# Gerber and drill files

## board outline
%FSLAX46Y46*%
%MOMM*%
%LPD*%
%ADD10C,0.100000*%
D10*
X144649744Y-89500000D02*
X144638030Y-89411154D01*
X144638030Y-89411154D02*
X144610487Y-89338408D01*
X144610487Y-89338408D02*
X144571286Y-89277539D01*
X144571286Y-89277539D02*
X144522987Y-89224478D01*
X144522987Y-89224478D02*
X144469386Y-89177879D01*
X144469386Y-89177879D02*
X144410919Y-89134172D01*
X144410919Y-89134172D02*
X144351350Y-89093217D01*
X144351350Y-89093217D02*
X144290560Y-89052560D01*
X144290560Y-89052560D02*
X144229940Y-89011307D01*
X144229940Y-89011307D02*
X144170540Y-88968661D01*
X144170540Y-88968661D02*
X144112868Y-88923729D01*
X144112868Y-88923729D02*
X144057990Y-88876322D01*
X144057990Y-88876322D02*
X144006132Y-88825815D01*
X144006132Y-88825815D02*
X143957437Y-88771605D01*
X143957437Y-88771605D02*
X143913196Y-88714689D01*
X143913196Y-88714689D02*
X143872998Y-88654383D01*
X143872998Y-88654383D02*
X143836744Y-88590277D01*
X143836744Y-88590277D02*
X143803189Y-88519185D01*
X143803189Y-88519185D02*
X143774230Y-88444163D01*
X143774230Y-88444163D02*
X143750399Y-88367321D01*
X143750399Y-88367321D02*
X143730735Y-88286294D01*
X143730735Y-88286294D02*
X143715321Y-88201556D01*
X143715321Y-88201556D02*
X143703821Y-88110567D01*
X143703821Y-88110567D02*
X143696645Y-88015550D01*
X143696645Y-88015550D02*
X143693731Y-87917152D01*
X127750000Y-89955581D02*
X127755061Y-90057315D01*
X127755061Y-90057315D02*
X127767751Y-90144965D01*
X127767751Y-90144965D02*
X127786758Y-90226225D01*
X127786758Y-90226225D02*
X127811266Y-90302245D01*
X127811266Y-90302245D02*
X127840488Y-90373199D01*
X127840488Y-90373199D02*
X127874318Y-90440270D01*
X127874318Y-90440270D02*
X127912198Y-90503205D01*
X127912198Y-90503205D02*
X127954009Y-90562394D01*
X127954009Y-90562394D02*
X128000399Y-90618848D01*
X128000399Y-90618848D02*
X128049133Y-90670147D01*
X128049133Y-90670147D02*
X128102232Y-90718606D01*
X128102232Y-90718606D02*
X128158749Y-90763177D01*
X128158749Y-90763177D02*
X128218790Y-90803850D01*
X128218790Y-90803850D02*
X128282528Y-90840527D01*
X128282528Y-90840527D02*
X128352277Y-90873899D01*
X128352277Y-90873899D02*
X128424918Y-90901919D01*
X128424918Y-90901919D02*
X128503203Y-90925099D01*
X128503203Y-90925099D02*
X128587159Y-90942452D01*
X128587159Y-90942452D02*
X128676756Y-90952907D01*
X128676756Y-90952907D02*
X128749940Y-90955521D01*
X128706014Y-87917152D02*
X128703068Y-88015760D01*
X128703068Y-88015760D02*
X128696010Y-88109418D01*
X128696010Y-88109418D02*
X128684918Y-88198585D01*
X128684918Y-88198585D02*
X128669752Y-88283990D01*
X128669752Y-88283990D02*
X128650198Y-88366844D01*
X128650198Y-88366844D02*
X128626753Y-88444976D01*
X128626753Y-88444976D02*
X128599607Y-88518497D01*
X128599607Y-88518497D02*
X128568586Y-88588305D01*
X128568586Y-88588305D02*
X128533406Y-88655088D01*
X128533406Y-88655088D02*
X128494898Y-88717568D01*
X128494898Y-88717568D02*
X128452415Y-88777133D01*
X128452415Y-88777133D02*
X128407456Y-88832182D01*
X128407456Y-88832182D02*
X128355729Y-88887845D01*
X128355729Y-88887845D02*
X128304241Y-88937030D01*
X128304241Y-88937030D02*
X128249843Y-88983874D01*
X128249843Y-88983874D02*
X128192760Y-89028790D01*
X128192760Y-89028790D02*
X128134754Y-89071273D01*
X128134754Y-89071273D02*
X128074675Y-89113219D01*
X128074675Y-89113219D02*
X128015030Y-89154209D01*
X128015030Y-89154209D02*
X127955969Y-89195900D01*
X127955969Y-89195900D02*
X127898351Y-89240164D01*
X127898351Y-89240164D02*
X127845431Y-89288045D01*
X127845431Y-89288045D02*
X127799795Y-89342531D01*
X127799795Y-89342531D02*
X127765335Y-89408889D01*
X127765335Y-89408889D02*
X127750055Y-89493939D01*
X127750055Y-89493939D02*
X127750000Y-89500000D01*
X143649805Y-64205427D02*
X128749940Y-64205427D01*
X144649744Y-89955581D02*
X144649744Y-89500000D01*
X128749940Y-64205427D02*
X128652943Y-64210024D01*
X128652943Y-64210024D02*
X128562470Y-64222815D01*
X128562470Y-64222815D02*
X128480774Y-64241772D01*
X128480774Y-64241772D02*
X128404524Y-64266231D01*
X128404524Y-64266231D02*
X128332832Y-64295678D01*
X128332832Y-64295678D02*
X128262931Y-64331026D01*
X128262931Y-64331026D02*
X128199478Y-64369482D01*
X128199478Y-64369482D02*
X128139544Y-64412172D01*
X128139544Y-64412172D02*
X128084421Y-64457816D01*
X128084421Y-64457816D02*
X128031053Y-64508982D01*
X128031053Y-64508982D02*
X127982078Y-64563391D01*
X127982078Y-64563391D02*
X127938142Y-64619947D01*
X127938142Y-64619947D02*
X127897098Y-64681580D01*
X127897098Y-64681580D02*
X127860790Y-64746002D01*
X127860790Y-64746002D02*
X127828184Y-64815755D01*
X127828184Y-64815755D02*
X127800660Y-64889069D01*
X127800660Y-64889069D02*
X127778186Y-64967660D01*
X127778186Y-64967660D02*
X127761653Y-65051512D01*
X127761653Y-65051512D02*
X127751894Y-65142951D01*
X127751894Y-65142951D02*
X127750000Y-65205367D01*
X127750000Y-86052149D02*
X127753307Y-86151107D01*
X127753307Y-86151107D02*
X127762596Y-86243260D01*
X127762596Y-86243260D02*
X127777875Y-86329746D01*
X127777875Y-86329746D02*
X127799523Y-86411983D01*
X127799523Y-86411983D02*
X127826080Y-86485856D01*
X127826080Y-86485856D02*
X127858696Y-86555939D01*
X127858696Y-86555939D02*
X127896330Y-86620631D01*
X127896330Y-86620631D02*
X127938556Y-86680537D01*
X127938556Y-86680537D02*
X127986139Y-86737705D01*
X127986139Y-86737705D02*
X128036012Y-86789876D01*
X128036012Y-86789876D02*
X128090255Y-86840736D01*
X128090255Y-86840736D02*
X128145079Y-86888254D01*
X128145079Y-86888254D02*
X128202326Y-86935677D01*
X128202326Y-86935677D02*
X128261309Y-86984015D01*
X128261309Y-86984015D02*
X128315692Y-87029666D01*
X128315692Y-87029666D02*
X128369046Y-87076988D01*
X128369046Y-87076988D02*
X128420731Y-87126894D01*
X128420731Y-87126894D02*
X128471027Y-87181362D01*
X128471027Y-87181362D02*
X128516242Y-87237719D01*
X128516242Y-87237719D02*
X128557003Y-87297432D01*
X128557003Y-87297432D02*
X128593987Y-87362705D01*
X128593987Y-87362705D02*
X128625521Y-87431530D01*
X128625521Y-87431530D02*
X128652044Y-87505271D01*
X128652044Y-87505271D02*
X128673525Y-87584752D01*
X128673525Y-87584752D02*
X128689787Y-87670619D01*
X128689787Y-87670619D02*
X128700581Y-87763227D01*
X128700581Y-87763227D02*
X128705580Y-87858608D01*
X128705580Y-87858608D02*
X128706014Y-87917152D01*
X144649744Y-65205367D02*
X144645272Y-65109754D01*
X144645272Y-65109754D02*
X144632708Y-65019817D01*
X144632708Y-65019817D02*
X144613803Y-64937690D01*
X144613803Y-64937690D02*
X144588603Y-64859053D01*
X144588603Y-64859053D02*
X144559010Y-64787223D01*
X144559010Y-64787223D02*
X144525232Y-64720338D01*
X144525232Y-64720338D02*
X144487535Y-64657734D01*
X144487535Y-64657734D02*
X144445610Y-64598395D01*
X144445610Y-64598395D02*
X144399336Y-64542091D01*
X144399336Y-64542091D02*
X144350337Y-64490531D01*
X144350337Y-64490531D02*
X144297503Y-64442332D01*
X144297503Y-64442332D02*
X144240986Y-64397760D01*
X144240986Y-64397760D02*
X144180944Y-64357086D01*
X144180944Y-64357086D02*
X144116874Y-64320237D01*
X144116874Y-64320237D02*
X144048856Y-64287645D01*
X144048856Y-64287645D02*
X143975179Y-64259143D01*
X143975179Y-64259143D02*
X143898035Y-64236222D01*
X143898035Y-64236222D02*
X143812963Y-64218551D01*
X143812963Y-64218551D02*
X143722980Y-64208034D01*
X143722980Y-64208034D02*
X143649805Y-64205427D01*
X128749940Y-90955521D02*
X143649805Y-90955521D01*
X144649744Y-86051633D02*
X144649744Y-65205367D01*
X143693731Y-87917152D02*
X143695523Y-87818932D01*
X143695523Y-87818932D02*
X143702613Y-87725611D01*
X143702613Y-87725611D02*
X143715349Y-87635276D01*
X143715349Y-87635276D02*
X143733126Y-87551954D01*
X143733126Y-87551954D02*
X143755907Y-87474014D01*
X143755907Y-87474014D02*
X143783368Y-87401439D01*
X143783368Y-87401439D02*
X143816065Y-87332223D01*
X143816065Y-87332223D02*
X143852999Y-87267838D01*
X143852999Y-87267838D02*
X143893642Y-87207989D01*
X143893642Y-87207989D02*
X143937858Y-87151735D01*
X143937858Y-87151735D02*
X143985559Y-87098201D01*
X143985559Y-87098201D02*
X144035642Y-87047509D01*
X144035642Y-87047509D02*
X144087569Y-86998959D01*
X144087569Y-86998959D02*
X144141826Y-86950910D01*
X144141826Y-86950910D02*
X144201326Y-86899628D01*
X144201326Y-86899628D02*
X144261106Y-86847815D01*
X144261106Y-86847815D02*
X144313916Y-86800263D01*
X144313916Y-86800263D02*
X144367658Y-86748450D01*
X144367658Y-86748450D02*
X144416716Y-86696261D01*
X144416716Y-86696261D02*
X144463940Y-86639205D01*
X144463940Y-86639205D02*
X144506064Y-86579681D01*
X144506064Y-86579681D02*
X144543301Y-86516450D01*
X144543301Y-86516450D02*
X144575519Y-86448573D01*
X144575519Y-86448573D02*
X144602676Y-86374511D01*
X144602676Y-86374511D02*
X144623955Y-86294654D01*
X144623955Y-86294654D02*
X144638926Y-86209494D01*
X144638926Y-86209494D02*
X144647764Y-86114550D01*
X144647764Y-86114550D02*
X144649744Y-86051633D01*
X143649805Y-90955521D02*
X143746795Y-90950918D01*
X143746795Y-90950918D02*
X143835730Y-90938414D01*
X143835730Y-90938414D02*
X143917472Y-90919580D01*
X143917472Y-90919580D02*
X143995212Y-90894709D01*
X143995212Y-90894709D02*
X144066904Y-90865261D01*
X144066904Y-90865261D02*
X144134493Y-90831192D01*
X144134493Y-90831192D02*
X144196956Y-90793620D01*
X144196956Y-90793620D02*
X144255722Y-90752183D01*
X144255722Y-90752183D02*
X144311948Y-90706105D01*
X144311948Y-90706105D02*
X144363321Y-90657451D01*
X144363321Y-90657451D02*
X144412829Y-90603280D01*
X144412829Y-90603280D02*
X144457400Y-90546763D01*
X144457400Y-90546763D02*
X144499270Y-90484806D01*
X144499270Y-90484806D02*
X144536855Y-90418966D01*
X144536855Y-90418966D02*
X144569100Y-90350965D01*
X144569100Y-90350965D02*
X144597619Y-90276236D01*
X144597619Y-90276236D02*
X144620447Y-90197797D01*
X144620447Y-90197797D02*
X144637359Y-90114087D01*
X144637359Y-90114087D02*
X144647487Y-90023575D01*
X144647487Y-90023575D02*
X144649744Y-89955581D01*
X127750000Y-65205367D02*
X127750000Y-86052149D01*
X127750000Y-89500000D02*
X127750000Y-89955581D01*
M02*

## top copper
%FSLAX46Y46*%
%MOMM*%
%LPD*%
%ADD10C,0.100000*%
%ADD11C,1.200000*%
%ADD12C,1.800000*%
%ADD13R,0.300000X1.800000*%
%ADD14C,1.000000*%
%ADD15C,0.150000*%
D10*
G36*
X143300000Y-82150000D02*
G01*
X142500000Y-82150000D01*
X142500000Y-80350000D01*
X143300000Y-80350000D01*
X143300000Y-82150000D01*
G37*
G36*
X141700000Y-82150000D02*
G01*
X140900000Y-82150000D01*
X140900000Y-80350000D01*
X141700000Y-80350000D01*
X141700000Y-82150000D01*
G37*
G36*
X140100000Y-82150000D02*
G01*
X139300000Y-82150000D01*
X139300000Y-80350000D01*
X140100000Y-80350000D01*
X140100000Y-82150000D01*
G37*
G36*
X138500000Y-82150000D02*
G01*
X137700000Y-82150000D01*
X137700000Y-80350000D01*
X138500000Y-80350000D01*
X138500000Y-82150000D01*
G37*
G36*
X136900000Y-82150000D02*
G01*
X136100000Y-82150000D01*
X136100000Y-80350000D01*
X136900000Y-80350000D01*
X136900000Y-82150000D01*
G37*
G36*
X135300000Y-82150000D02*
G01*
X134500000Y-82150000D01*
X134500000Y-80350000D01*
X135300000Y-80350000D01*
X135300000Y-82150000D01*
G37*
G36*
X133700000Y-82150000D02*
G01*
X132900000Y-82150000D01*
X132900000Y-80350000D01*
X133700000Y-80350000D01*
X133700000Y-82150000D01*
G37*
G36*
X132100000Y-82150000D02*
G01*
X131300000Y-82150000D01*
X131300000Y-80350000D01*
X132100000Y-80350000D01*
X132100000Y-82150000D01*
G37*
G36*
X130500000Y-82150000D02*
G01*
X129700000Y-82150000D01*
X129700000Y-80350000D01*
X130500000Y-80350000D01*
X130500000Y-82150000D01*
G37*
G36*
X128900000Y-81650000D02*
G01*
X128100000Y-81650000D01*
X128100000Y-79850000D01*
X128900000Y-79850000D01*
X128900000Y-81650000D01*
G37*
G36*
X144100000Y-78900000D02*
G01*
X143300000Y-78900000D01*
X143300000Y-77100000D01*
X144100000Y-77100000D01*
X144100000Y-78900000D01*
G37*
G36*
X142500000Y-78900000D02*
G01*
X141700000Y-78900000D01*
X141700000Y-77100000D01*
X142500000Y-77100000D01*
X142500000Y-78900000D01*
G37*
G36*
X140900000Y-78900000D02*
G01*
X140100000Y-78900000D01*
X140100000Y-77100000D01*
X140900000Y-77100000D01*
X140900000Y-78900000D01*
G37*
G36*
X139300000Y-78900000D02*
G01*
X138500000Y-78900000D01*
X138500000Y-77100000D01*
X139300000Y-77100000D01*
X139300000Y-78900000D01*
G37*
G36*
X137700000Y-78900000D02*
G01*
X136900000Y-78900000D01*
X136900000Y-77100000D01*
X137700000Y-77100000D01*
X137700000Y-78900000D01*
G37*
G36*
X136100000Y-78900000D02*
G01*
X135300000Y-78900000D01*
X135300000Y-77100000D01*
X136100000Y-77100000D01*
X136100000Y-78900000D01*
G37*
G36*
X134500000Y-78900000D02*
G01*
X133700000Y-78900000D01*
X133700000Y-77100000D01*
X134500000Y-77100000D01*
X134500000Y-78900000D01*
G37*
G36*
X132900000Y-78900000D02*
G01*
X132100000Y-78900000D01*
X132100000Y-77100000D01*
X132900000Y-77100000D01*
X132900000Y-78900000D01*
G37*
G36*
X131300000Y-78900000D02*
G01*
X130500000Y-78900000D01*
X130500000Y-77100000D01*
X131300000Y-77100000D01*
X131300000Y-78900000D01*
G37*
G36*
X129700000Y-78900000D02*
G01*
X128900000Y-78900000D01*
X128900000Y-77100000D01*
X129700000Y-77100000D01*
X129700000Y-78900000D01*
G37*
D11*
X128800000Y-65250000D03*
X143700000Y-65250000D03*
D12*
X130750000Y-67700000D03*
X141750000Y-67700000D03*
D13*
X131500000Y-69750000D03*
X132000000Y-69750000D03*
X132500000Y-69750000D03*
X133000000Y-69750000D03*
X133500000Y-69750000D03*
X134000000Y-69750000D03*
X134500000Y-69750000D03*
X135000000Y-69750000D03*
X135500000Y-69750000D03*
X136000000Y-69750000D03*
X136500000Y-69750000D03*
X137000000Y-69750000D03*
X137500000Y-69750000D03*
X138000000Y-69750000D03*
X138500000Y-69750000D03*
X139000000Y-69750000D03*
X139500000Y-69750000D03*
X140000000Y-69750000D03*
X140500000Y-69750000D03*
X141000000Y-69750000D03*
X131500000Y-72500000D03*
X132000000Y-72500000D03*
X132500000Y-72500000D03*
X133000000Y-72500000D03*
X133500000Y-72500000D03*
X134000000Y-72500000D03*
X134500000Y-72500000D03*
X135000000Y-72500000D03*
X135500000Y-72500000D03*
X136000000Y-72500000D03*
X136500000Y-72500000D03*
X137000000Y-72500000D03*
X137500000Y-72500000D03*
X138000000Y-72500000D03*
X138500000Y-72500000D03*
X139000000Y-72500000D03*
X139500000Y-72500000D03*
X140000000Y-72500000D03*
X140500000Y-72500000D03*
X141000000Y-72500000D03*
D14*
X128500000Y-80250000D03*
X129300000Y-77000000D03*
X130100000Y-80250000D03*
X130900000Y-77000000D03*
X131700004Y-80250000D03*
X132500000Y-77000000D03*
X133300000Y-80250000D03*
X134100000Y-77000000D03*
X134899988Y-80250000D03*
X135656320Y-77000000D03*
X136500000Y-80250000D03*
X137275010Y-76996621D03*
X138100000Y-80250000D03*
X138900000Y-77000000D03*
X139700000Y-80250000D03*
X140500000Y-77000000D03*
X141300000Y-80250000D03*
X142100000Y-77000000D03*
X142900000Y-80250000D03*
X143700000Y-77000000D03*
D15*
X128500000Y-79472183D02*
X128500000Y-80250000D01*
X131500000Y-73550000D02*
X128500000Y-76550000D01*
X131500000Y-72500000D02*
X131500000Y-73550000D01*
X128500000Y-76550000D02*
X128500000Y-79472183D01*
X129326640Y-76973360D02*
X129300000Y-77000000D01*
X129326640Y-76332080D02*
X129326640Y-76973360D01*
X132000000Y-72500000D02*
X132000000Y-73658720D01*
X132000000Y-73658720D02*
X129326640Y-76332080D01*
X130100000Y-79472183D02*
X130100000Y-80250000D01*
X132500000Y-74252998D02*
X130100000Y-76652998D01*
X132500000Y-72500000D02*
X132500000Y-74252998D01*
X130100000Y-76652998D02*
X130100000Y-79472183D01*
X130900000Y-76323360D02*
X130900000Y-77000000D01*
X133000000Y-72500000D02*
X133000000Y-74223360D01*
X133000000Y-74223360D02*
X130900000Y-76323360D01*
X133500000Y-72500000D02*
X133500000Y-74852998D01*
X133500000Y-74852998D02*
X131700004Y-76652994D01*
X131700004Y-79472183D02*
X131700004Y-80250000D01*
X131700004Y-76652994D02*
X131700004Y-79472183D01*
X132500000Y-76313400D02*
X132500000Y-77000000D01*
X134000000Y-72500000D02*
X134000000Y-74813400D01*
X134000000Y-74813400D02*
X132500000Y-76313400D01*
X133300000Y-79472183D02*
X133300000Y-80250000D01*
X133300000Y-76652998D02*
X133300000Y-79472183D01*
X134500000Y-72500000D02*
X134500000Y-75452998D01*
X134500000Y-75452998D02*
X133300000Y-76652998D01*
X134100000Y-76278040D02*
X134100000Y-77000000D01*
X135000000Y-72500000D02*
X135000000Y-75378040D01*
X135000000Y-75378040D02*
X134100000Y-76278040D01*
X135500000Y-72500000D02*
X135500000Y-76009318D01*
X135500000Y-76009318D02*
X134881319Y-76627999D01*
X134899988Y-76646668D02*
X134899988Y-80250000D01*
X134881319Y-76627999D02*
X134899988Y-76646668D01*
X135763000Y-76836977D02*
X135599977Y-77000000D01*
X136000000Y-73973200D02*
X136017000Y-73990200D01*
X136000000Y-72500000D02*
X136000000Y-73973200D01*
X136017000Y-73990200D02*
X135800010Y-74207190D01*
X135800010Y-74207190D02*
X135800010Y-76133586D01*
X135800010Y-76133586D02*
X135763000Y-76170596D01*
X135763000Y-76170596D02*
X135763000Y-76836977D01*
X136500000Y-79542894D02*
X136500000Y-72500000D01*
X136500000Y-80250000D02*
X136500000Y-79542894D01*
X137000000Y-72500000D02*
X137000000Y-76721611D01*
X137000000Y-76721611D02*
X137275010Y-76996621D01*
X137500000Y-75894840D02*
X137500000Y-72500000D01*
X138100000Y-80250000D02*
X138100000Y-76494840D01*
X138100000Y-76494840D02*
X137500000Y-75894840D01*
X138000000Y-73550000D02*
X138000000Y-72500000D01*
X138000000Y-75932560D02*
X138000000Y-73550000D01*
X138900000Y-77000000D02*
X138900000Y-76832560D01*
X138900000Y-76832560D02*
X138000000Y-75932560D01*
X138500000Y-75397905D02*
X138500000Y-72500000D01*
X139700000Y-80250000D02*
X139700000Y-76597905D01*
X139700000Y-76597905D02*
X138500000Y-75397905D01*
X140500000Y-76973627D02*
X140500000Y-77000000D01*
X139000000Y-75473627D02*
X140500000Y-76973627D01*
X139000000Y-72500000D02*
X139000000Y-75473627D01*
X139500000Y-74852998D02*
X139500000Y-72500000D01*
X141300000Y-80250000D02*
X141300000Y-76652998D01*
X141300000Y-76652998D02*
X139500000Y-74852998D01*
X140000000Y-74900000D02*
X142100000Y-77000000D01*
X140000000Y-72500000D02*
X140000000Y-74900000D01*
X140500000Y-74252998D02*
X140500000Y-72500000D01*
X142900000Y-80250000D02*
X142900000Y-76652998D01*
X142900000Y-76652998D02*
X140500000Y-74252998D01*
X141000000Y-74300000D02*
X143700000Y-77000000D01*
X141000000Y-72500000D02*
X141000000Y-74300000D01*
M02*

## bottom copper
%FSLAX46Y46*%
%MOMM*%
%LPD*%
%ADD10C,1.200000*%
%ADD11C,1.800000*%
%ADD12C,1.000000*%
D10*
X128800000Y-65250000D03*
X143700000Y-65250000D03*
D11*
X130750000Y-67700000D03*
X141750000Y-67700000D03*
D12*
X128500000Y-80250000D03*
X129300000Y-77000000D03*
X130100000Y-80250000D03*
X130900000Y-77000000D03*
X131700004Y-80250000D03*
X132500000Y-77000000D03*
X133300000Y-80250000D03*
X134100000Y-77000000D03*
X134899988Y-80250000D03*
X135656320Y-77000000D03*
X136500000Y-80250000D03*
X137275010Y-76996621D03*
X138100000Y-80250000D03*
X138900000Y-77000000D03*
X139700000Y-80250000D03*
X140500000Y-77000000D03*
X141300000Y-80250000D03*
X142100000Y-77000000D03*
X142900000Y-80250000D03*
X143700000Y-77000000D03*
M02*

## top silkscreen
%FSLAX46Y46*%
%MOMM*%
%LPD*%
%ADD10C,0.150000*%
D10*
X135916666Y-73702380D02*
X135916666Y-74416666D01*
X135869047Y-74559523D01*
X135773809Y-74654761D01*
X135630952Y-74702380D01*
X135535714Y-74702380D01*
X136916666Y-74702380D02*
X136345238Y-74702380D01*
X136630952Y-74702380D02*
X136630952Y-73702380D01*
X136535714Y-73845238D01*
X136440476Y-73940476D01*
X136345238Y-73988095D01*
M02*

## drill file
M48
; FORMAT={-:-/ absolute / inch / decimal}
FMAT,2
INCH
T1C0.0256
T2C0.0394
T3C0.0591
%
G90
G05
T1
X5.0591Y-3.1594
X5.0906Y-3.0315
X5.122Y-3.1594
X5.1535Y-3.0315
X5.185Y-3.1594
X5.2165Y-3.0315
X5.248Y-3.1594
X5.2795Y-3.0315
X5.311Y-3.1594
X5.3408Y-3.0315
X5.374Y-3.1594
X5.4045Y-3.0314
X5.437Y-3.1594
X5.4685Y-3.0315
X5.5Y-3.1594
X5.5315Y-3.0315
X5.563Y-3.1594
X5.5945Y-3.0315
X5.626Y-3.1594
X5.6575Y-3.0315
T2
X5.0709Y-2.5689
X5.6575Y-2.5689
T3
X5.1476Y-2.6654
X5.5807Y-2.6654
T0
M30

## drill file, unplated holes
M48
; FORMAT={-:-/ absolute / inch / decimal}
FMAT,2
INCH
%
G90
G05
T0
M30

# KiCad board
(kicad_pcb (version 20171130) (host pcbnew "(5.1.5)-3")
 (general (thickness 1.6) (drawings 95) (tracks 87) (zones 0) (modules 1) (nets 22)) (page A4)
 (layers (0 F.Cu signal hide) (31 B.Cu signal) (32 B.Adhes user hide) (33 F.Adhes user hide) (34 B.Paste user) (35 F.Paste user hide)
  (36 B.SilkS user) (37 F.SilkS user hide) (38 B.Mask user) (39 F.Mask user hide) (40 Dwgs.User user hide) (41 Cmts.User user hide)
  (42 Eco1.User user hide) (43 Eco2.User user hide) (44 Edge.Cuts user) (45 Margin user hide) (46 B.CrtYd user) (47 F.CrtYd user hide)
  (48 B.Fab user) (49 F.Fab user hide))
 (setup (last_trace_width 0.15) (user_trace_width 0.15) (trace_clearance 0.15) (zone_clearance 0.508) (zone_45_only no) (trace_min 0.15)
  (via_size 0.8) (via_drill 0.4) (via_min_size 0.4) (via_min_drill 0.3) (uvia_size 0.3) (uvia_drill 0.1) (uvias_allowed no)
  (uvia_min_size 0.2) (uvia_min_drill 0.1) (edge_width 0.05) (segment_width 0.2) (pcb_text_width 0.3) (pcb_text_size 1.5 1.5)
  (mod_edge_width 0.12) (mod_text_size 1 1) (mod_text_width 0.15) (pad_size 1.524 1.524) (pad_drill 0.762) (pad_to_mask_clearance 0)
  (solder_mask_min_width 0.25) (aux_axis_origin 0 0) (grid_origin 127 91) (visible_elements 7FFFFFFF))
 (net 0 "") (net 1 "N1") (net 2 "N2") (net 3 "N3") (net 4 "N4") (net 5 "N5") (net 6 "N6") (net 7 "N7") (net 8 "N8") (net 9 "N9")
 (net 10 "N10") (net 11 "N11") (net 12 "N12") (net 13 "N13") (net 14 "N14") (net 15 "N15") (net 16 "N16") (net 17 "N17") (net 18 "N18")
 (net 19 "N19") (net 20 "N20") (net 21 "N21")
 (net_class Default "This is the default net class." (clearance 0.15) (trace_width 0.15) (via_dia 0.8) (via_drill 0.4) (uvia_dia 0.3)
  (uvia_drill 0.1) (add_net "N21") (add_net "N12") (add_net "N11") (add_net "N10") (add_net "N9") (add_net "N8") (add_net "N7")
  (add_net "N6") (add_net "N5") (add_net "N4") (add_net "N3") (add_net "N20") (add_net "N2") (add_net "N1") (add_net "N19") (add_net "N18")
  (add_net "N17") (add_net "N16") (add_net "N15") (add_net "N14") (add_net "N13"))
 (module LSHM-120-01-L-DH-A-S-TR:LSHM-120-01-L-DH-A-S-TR (layer F.Cu) (at 136.25 69.75 180)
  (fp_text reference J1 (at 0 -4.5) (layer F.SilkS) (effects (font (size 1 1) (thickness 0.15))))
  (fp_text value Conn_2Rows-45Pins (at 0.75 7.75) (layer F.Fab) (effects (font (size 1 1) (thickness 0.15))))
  (pad 44 thru_hole circle (at 7.45 4.5 270) (size 1.2 1.2) (drill 1) (layers *.Cu *.Mask) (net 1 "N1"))
  (pad 43 thru_hole circle (at -7.45 4.5 270) (size 1.2 1.2) (drill 1) (layers *.Cu *.Mask) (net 1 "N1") (solder_paste_margin -0.5))
  (pad 42 thru_hole circle (at 5.5 2.05 270) (size 1.8 1.8) (drill 1.5) (layers *.Cu *.Mask) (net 1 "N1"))
  (pad 41 thru_hole circle (at -5.5 2.05 270) (size 1.8 1.8) (drill 1.5) (layers *.Cu *.Mask) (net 1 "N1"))
  (pad 40 smd rect (at 4.75 0 270) (size 1.8 0.3) (layers F.Cu F.Paste F.Mask) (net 1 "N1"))
  (pad 39 smd rect (at 4.25 0 270) (size 1.8 0.3) (layers F.Cu F.Paste F.Mask) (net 1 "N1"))
  (pad 38 smd rect (at 3.75 0 270) (size 1.8 0.3) (layers F.Cu F.Paste F.Mask) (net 1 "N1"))
  (pad 37 smd rect (at 3.25 0 270) (size 1.8 0.3) (layers F.Cu F.Paste F.Mask) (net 1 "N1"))
  (pad 36 smd rect (at 2.75 0 270) (size 1.8 0.3) (layers F.Cu F.Paste F.Mask) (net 1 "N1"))
  (pad 35 smd rect (at 2.25 0 270) (size 1.8 0.3) (layers F.Cu F.Paste F.Mask) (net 1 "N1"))
  (pad 34 smd rect (at 1.75 0 270) (size 1.8 0.3) (layers F.Cu F.Paste F.Mask) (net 1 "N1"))
  (pad 33 smd rect (at 1.25 0 270) (size 1.8 0.3) (layers F.Cu F.Paste F.Mask) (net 1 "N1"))
  (pad 32 smd rect (at 0.75 0 270) (size 1.8 0.3) (layers F.Cu F.Paste F.Mask) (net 1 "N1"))
  (pad 31 smd rect (at 0.25 0 270) (size 1.8 0.3) (layers F.Cu F.Paste F.Mask) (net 1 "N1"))
  (pad 30 smd rect (at -0.25 0 270) (size 1.8 0.3) (layers F.Cu F.Paste F.Mask) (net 1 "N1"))
  (pad 29 smd rect (at -0.75 0 270) (size 1.8 0.3) (layers F.Cu F.Paste F.Mask) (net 1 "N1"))
  (pad 28 smd rect (at -1.25 0 270) (size 1.8 0.3) (layers F.Cu F.Paste F.Mask) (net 1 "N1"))
  (pad 27 smd rect (at -1.75 0 270) (size 1.8 0.3) (layers F.Cu F.Paste F.Mask) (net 1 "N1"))
  (pad 26 smd rect (at -2.25 0 270) (size 1.8 0.3) (layers F.Cu F.Paste F.Mask) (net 1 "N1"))
  (pad 25 smd rect (at -2.75 0 270) (size 1.8 0.3) (layers F.Cu F.Paste F.Mask) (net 1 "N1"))
  (pad 24 smd rect (at -3.25 0 270) (size 1.8 0.3) (layers F.Cu F.Paste F.Mask) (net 1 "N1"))
  (pad 23 smd rect (at -3.75 0 270) (size 1.8 0.3) (layers F.Cu F.Paste F.Mask) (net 1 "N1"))
  (pad 22 smd rect (at -4.25 0 270) (size 1.8 0.3) (layers F.Cu F.Paste F.Mask) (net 1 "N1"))
  (pad 21 smd rect (at -4.75 0 270) (size 1.8 0.3) (layers F.Cu F.Paste F.Mask) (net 1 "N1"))
  (pad 20 smd rect (at 4.75 -2.75 270) (size 1.8 0.3) (layers F.Cu F.Paste F.Mask) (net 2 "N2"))
  (pad 19 smd rect (at 4.25 -2.75 270) (size 1.8 0.3) (layers F.Cu F.Paste F.Mask) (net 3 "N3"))
  (pad 18 smd rect (at 3.75 -2.75 270) (size 1.8 0.3) (layers F.Cu F.Paste F.Mask) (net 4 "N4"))
  (pad 17 smd rect (at 3.25 -2.75 270) (size 1.8 0.3) (layers F.Cu F.Paste F.Mask) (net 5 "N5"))
  (pad 16 smd rect (at 2.75 -2.75 270) (size 1.8 0.3) (layers F.Cu F.Paste F.Mask) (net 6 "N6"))
  (pad 15 smd rect (at 2.25 -2.75 270) (size 1.8 0.3) (layers F.Cu F.Paste F.Mask) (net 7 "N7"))
  (pad 14 smd rect (at 1.75 -2.75 270) (size 1.8 0.3) (layers F.Cu F.Paste F.Mask) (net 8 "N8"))
  (pad 13 smd rect (at 1.25 -2.75 270) (size 1.8 0.3) (layers F.Cu F.Paste F.Mask) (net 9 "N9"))
  (pad 12 smd rect (at 0.75 -2.75 270) (size 1.8 0.3) (layers F.Cu F.Paste F.Mask) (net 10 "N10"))
  (pad 11 smd rect (at 0.25 -2.75 270) (size 1.8 0.3) (layers F.Cu F.Paste F.Mask) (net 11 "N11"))
  (pad 10 smd rect (at -0.25 -2.75 270) (size 1.8 0.3) (layers F.Cu F.Paste F.Mask) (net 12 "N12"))
  (pad 9 smd rect (at -0.75 -2.75 270) (size 1.8 0.3) (layers F.Cu F.Paste F.Mask) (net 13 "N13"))
  (pad 8 smd rect (at -1.25 -2.75 270) (size 1.8 0.3) (layers F.Cu F.Paste F.Mask) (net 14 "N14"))
  (pad 7 smd rect (at -1.75 -2.75 270) (size 1.8 0.3) (layers F.Cu F.Paste F.Mask) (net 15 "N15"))
  (pad 6 smd rect (at -2.25 -2.75 270) (size 1.8 0.3) (layers F.Cu F.Paste F.Mask) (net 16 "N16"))
  (pad 5 smd rect (at -2.75 -2.75 270) (size 1.8 0.3) (layers F.Cu F.Paste F.Mask) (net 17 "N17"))
  (pad 4 smd rect (at -3.25 -2.75 270) (size 1.8 0.3) (layers F.Cu F.Paste F.Mask) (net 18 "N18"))
  (pad 3 smd rect (at -3.75 -2.75 270) (size 1.8 0.3) (layers F.Cu F.Paste F.Mask) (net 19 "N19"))
  (pad 2 smd rect (at -4.25 -2.75 270) (size 1.8 0.3) (layers F.Cu F.Paste F.Mask) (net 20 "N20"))
  (pad 1 smd rect (at -4.75 -2.75 270) (size 1.8 0.3) (layers F.Cu F.Paste F.Mask) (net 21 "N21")))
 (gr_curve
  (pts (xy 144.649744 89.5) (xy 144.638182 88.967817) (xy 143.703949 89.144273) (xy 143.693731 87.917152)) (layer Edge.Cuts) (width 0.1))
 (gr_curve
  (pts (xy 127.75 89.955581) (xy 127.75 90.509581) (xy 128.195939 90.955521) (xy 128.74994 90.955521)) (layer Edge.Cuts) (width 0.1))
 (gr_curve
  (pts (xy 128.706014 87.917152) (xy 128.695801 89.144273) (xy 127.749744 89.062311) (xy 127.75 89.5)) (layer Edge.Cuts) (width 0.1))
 (gr_line (start 143.649805 64.205427) (end 128.74994 64.205427) (layer Edge.Cuts) (width 0.1))
 (gr_line (start 144.649744 89.955581) (end 144.649744 89.5) (layer Edge.Cuts) (width 0.1))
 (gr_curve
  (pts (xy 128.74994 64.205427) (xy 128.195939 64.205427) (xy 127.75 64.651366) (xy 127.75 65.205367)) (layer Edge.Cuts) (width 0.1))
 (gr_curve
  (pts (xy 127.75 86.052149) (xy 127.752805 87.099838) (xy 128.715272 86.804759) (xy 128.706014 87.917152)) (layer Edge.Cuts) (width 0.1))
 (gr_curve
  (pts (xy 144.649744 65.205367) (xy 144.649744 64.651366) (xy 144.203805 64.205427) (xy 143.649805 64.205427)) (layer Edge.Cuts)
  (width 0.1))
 (gr_line (start 128.74994 90.955521) (end 143.649805 90.955521) (layer Edge.Cuts) (width 0.1))
 (gr_line (start 144.649744 86.051633) (end 144.649744 65.205367) (layer Edge.Cuts) (width 0.1))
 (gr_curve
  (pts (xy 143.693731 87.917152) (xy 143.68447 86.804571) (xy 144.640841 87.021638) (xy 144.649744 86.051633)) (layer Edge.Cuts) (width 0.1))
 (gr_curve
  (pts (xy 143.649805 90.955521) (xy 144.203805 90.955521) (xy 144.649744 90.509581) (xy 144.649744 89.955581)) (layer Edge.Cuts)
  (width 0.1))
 (gr_line (start 127.75 65.205367) (end 127.75 86.052149) (layer Edge.Cuts) (width 0.1))
 (gr_line (start 127.75 89.5) (end 127.75 89.955581) (layer Edge.Cuts) (width 0.1))
 (gr_poly (pts (xy 142.5 80.35) (xy 142.5 82.15) (xy 143.3 82.15) (xy 143.3 80.35)) (layer F.Cu) (width 0))
 (gr_poly (pts (xy 140.9 80.35) (xy 140.9 82.15) (xy 141.7 82.15) (xy 141.7 80.35)) (layer F.Cu) (width 0))
 (gr_poly (pts (xy 139.3 80.35) (xy 139.3 82.15) (xy 140.1 82.15) (xy 140.1 80.35)) (layer F.Cu) (width 0))
 (gr_poly (pts (xy 137.7 80.35) (xy 137.7 82.15) (xy 138.5 82.15) (xy 138.5 80.35)) (layer F.Cu) (width 0))
 (gr_poly (pts (xy 136.1 80.35) (xy 136.1 82.15) (xy 136.9 82.15) (xy 136.9 80.35)) (layer F.Cu) (width 0))
 (gr_poly (pts (xy 134.5 80.35) (xy 134.5 82.15) (xy 135.3 82.15) (xy 135.3 80.35)) (layer F.Cu) (width 0))
 (gr_poly (pts (xy 132.9 80.35) (xy 132.9 82.15) (xy 133.7 82.15) (xy 133.7 80.35)) (layer F.Cu) (width 0))
 (gr_poly (pts (xy 131.3 80.35) (xy 131.3 82.15) (xy 132.1 82.15) (xy 132.1 80.35)) (layer F.Cu) (width 0))
 (gr_poly (pts (xy 129.7 80.35) (xy 129.7 82.15) (xy 130.5 82.15) (xy 130.5 80.35)) (layer F.Cu) (width 0))
 (gr_poly (pts (xy 128.1 79.85) (xy 128.1 81.65) (xy 128.9 81.65) (xy 128.9 79.85)) (layer F.Cu) (width 0))
 (gr_poly (pts (xy 143.3 77.1) (xy 143.3 78.9) (xy 144.1 78.9) (xy 144.1 77.1)) (layer F.Cu) (width 0))
 (gr_poly (pts (xy 141.7 77.1) (xy 141.7 78.9) (xy 142.5 78.9) (xy 142.5 77.1)) (layer F.Cu) (width 0))
 (gr_poly (pts (xy 140.1 77.1) (xy 140.1 78.9) (xy 140.9 78.9) (xy 140.9 77.1)) (layer F.Cu) (width 0))
 (gr_poly (pts (xy 138.5 77.1) (xy 138.5 78.9) (xy 139.3 78.9) (xy 139.3 77.1)) (layer F.Cu) (width 0))
 (gr_poly (pts (xy 136.9 77.1) (xy 136.9 78.9) (xy 137.7 78.9) (xy 137.7 77.1)) (layer F.Cu) (width 0))
 (gr_poly (pts (xy 135.3 77.1) (xy 135.3 78.9) (xy 136.1 78.9) (xy 136.1 77.1)) (layer F.Cu) (width 0))
 (gr_poly (pts (xy 133.7 77.1) (xy 133.7 78.9) (xy 134.5 78.9) (xy 134.5 77.1)) (layer F.Cu) (width 0))
 (gr_poly (pts (xy 132.1 77.1) (xy 132.1 78.9) (xy 132.9 78.9) (xy 132.9 77.1)) (layer F.Cu) (width 0))
 (gr_poly (pts (xy 130.5 77.1) (xy 130.5 78.9) (xy 131.3 78.9) (xy 131.3 77.1)) (layer F.Cu) (width 0))
 (gr_poly (pts (xy 128.9 77.1) (xy 128.9 78.9) (xy 129.7 78.9) (xy 129.7 77.1)) (layer F.Cu) (width 0))
 (via (at 128.5 80.25) (size 1) (drill 0.65) (layers F.Cu B.Cu) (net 2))
 (segment (start 128.5 79.472183) (end 128.5 80.25) (width 0.15) (layer F.Cu) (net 2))
 (segment (start 131.5 73.55) (end 128.5 76.55) (width 0.15) (layer F.Cu) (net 2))
 (segment (start 131.5 72.5) (end 131.5 73.55) (width 0.15) (layer F.Cu) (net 2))
 (segment (start 128.5 76.55) (end 128.5 79.472183) (width 0.15) (layer F.Cu) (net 2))
 (via (at 129.3 77) (size 1) (drill 0.65) (layers F.Cu B.Cu) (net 3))
 (segment (start 129.32664 76.97336) (end 129.3 77) (width 0.15) (layer F.Cu) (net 3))
 (segment (start 129.32664 76.33208) (end 129.32664 76.97336) (width 0.15) (layer F.Cu) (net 3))
 (segment (start 132 72.5) (end 132 73.65872) (width 0.15) (layer F.Cu) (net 3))
 (segment (start 132 73.65872) (end 129.32664 76.33208) (width 0.15) (layer F.Cu) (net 3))
 (via (at 130.1 80.25) (size 1) (drill 0.65) (layers F.Cu B.Cu) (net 4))
 (segment (start 130.1 79.472183) (end 130.1 80.25) (width 0.15) (layer F.Cu) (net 4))
 (segment (start 132.5 74.252998) (end 130.1 76.652998) (width 0.15) (layer F.Cu) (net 4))
 (segment (start 132.5 72.5) (end 132.5 74.252998) (width 0.15) (layer F.Cu) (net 4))
 (segment (start 130.1 76.652998) (end 130.1 79.472183) (width 0.15) (layer F.Cu) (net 4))
 (via (at 130.9 77) (size 1) (drill 0.65) (layers F.Cu B.Cu) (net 5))
 (segment (start 130.9 76.32336) (end 130.9 77) (width 0.15) (layer F.Cu) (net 5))
 (segment (start 133 72.5) (end 133 74.22336) (width 0.15) (layer F.Cu) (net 5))
 (segment (start 133 74.22336) (end 130.9 76.32336) (width 0.15) (layer F.Cu) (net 5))
 (via (at 131.700004 80.25) (size 1) (drill 0.65) (layers F.Cu B.Cu) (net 6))
 (segment (start 133.5 72.5) (end 133.5 74.852998) (width 0.15) (layer F.Cu) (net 6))
 (segment (start 133.5 74.852998) (end 131.700004 76.652994) (width 0.15) (layer F.Cu) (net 6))
 (segment (start 131.700004 79.472183) (end 131.700004 80.25) (width 0.15) (layer F.Cu) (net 6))
 (segment (start 131.700004 76.652994) (end 131.700004 79.472183) (width 0.15) (layer F.Cu) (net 6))
 (via (at 132.5 77) (size 1) (drill 0.65) (layers F.Cu B.Cu) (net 7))
 (segment (start 132.5 76.3134) (end 132.5 77) (width 0.15) (layer F.Cu) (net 7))
 (segment (start 134 72.5) (end 134 74.8134) (width 0.15) (layer F.Cu) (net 7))
 (segment (start 134 74.8134) (end 132.5 76.3134) (width 0.15) (layer F.Cu) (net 7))
 (via (at 133.3 80.25) (size 1) (drill 0.65) (layers F.Cu B.Cu) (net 8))
 (segment (start 133.3 79.472183) (end 133.3 80.25) (width 0.15) (layer F.Cu) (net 8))
 (segment (start 133.3 76.652998) (end 133.3 79.472183) (width 0.15) (layer F.Cu) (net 8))
 (segment (start 134.5 72.5) (end 134.5 75.452998) (width 0.15) (layer F.Cu) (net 8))
 (segment (start 134.5 75.452998) (end 133.3 76.652998) (width 0.15) (layer F.Cu) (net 8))
 (via (at 134.1 77) (size 1) (drill 0.65) (layers F.Cu B.Cu) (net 9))
 (segment (start 134.1 76.27804) (end 134.1 77) (width 0.15) (layer F.Cu) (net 9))
 (segment (start 135 72.5) (end 135 75.37804) (width 0.15) (layer F.Cu) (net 9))
 (segment (start 135 75.37804) (end 134.1 76.27804) (width 0.15) (layer F.Cu) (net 9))
 (via (at 134.899988 80.25) (size 1) (drill 0.65) (layers F.Cu B.Cu) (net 10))
 (segment (start 135.5 72.5) (end 135.5 76.009318) (width 0.15) (layer F.Cu) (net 10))
 (segment (start 135.5 76.009318) (end 134.881319 76.627999) (width 0.15) (layer F.Cu) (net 10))
 (segment (start 134.899988 76.646668) (end 134.899988 80.25) (width 0.15) (layer F.Cu) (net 10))
 (segment (start 134.881319 76.627999) (end 134.899988 76.646668) (width 0.15) (layer F.Cu) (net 10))
 (via (at 135.65632 77) (size 1) (drill 0.65) (layers F.Cu B.Cu) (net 11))
 (segment (start 135.763 76.836977) (end 135.599977 77) (width 0.15) (layer F.Cu) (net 11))
 (segment (start 136 73.9732) (end 136.017 73.9902) (width 0.15) (layer F.Cu) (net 11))
 (segment (start 136 72.5) (end 136 73.9732) (width 0.15) (layer F.Cu) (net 11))
 (segment (start 136.017 73.9902) (end 135.80001 74.20719) (width 0.15) (layer F.Cu) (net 11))
 (segment (start 135.80001 74.20719) (end 135.80001 76.133586) (width 0.15) (layer F.Cu) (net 11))
 (segment (start 135.80001 76.133586) (end 135.763 76.170596) (width 0.15) (layer F.Cu) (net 11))
 (segment (start 135.763 76.170596) (end 135.763 76.836977) (width 0.15) (layer F.Cu) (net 11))
 (via (at 136.5 80.25) (size 1) (drill 0.65) (layers F.Cu B.Cu) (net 12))
 (segment (start 136.5 79.542894) (end 136.5 72.5) (width 0.15) (layer F.Cu) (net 12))
 (segment (start 136.5 80.25) (end 136.5 79.542894) (width 0.15) (layer F.Cu) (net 12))
 (segment (start 137 72.5) (end 137 76.721611) (width 0.15) (layer F.Cu) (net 13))
 (segment (start 137 76.721611) (end 137.27501 76.996621) (width 0.15) (layer F.Cu) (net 13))
 (via (at 137.27501 76.996621) (size 1) (drill 0.65) (layers F.Cu B.Cu) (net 13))
 (via (at 138.1 80.25) (size 1) (drill 0.65) (layers F.Cu B.Cu) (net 14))
 (segment (start 137.5 75.89484) (end 137.5 72.5) (width 0.15) (layer F.Cu) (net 14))
 (segment (start 138.1 80.25) (end 138.1 76.49484) (width 0.15) (layer F.Cu) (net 14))
 (segment (start 138.1 76.49484) (end 137.5 75.89484) (width 0.15) (layer F.Cu) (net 14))
 (via (at 138.9 77) (size 1) (drill 0.65) (layers F.Cu B.Cu) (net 15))
 (segment (start 138 73.55) (end 138 72.5) (width 0.15) (layer F.Cu) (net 15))
 (segment (start 138 75.93256) (end 138 73.55) (width 0.15) (layer F.Cu) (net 15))
 (segment (start 138.9 77) (end 138.9 76.83256) (width 0.15) (layer F.Cu) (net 15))
 (segment (start 138.9 76.83256) (end 138 75.93256) (width 0.15) (layer F.Cu) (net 15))
 (via (at 139.7 80.25) (size 1) (drill 0.65) (layers F.Cu B.Cu) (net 16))
 (segment (start 138.5 75.397905) (end 138.5 72.5) (width 0.15) (layer F.Cu) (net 16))
 (segment (start 139.7 80.25) (end 139.7 76.597905) (width 0.15) (layer F.Cu) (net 16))
 (segment (start 139.7 76.597905) (end 138.5 75.397905) (width 0.15) (layer F.Cu) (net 16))
 (via (at 140.5 77) (size 1) (drill 0.65) (layers F.Cu B.Cu) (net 17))
 (segment (start 140.5 76.973627) (end 140.5 77) (width 0.15) (layer F.Cu) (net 17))
 (segment (start 139 75.473627) (end 140.5 76.973627) (width 0.15) (layer F.Cu) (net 17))
 (segment (start 139 72.5) (end 139 75.473627) (width 0.15) (layer F.Cu) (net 17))
 (via (at 141.3 80.25) (size 1) (drill 0.65) (layers F.Cu B.Cu) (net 18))
 (segment (start 139.5 74.852998) (end 139.5 72.5) (width 0.15) (layer F.Cu) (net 18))
 (segment (start 141.3 80.25) (end 141.3 76.652998) (width 0.15) (layer F.Cu) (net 18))
 (segment (start 141.3 76.652998) (end 139.5 74.852998) (width 0.15) (layer F.Cu) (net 18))
 (via (at 142.1 77) (size 1) (drill 0.65) (layers F.Cu B.Cu) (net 19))
 (segment (start 140 74.9) (end 142.1 77) (width 0.15) (layer F.Cu) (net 19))
 (segment (start 140 72.5) (end 140 74.9) (width 0.15) (layer F.Cu) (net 19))
 (via (at 142.9 80.25) (size 1) (drill 0.65) (layers F.Cu B.Cu) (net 20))
 (segment (start 140.5 74.252998) (end 140.5 72.5) (width 0.15) (layer F.Cu) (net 20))
 (segment (start 142.9 80.25) (end 142.9 76.652998) (width 0.15) (layer F.Cu) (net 20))
 (segment (start 142.9 76.652998) (end 140.5 74.252998) (width 0.15) (layer F.Cu) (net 20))
 (via (at 143.7 77) (size 1) (drill 0.65) (layers F.Cu B.Cu) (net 21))
 (segment (start 141 74.3) (end 143.7 77) (width 0.15) (layer F.Cu) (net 21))
 (segment (start 141 72.5) (end 141 74.3) (width 0.15) (layer F.Cu) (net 21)))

